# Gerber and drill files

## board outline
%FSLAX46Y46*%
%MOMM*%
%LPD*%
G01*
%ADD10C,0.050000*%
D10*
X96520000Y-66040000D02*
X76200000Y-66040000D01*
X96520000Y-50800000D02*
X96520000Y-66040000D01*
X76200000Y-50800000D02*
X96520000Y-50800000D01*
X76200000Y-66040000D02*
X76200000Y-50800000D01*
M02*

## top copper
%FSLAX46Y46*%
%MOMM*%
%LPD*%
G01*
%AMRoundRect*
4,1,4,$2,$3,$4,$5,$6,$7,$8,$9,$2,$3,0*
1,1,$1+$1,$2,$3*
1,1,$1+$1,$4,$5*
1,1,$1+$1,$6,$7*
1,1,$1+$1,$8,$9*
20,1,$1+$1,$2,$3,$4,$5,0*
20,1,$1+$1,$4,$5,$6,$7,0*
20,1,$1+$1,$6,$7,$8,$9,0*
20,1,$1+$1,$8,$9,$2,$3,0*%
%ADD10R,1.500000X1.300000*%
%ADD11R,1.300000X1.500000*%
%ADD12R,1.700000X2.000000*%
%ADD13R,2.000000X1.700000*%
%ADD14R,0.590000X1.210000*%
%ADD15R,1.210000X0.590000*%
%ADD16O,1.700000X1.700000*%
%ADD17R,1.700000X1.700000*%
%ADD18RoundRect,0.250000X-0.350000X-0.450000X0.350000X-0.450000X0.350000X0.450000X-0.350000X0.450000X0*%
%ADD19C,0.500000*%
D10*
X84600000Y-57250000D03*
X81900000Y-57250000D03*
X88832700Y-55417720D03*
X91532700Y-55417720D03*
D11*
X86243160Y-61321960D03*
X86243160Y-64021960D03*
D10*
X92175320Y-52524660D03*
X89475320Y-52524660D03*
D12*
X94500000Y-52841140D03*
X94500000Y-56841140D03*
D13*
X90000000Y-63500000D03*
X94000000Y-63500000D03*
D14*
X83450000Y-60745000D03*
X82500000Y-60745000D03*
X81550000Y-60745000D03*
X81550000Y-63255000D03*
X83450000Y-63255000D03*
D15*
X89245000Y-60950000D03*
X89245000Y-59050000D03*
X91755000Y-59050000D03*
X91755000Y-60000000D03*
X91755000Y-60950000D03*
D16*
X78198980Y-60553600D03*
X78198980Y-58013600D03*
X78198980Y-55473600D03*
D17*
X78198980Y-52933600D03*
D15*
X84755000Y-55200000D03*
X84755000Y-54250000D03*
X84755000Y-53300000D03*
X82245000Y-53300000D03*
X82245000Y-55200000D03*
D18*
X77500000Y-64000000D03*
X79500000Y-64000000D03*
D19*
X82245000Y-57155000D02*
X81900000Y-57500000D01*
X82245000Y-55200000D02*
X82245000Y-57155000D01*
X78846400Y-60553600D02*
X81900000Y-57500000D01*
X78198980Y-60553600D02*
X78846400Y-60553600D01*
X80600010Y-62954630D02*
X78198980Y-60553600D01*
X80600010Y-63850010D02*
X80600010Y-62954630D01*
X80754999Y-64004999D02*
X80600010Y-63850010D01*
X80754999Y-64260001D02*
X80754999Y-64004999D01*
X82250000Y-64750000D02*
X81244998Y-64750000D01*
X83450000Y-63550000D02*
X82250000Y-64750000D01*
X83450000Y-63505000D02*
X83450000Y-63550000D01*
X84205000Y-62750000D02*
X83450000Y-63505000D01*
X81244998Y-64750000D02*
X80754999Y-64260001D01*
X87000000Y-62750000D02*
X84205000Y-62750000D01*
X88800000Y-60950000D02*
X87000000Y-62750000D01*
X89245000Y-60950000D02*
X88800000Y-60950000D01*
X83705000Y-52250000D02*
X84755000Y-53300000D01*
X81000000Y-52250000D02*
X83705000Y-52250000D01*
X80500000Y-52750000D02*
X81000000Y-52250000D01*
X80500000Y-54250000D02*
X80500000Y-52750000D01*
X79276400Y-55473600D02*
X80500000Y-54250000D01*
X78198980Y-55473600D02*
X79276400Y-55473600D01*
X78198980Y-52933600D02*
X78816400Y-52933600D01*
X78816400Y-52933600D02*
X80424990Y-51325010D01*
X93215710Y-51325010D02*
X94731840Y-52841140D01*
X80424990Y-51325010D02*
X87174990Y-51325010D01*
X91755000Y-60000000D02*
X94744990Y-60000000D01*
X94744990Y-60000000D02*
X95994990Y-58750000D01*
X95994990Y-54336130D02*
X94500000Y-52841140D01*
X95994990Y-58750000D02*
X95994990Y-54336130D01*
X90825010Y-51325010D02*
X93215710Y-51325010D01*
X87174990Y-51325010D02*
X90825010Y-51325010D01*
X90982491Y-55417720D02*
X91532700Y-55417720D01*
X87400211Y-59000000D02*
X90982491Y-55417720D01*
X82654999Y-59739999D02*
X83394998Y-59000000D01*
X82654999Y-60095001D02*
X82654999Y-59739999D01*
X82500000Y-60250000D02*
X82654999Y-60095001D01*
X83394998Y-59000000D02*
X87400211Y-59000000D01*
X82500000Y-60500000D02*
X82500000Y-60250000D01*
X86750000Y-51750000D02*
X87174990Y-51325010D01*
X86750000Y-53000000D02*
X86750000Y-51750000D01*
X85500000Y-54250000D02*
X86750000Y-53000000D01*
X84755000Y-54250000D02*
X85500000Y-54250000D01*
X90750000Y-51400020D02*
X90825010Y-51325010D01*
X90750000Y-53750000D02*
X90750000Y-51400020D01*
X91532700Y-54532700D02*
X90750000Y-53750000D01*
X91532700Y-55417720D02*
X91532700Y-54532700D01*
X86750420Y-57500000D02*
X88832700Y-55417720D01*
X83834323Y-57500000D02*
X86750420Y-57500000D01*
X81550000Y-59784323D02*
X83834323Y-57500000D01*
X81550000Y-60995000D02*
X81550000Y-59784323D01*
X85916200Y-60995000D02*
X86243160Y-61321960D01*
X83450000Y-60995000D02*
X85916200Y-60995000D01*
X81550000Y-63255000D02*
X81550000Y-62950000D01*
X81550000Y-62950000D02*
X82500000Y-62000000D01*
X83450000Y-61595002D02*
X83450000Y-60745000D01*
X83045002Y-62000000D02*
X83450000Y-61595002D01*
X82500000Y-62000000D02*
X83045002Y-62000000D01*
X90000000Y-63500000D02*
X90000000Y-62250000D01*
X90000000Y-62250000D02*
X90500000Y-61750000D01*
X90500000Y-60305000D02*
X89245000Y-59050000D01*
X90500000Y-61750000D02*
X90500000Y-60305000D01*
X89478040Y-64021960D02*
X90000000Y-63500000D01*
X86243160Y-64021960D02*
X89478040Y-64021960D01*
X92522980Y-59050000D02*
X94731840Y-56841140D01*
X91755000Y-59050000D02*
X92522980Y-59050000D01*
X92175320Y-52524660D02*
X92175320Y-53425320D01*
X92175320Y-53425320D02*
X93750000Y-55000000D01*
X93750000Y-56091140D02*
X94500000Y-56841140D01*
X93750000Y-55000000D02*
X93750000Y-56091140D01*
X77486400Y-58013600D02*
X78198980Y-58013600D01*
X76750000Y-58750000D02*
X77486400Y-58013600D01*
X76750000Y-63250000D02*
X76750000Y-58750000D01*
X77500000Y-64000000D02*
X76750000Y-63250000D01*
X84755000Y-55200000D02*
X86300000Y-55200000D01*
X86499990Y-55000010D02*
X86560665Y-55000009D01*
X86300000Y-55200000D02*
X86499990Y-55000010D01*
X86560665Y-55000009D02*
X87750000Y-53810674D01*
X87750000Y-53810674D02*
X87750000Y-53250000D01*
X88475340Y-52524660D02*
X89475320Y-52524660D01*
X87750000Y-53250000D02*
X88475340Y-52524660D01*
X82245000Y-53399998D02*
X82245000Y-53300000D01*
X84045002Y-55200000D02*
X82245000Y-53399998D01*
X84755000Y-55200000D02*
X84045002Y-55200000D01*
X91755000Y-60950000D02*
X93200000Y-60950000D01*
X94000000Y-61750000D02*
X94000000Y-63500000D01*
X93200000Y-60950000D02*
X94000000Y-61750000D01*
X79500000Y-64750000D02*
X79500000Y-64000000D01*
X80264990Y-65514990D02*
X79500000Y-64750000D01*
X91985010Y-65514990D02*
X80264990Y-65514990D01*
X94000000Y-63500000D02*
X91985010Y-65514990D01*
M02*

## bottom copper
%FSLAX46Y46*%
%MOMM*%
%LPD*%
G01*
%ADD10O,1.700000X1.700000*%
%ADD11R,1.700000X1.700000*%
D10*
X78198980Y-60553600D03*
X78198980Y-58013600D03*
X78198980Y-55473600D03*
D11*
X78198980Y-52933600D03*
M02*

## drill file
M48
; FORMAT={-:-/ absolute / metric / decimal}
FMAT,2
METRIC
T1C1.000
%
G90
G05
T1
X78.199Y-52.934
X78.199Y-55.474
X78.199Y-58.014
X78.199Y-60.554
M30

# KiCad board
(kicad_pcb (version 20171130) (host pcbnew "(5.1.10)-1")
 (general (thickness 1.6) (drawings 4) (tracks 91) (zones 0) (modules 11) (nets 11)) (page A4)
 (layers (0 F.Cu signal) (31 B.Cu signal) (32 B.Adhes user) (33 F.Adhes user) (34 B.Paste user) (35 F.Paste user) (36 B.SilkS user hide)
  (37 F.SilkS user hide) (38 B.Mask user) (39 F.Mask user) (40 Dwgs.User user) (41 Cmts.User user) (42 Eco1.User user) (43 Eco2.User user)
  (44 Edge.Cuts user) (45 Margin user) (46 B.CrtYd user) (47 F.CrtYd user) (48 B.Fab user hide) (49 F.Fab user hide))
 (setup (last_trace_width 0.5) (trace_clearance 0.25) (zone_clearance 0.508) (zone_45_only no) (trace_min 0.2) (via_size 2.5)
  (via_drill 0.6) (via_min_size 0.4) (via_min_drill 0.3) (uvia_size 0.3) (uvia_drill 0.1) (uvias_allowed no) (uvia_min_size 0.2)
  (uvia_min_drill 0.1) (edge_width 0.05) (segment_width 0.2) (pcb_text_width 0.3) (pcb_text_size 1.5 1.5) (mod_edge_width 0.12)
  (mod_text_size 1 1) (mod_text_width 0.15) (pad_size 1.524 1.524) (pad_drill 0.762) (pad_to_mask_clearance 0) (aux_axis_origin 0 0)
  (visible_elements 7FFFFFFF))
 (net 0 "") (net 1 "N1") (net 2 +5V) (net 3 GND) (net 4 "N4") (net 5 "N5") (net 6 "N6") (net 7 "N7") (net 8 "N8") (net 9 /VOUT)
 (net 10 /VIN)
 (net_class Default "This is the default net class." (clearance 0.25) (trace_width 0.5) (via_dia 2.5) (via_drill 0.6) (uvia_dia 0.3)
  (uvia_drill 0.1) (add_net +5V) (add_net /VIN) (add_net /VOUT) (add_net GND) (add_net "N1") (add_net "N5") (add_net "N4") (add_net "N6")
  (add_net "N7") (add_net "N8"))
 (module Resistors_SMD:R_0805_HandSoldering (layer F.Cu) (at 83.25 57.25)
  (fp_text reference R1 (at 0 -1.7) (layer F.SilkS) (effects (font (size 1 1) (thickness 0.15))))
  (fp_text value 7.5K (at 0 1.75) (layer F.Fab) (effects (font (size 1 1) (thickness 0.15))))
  (pad 2 smd rect (at 1.35 0) (size 1.5 1.3) (layers F.Cu F.Paste F.Mask) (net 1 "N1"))
  (pad 1 smd rect (at -1.35 0) (size 1.5 1.3) (layers F.Cu F.Paste F.Mask) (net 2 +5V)))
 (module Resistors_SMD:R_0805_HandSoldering (layer F.Cu) (at 90.1827 55.41772)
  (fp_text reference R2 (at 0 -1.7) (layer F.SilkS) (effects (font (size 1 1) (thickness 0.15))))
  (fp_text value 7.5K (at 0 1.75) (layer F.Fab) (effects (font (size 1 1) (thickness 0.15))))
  (pad 1 smd rect (at -1.35 0) (size 1.5 1.3) (layers F.Cu F.Paste F.Mask) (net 1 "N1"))
  (pad 2 smd rect (at 1.35 0) (size 1.5 1.3) (layers F.Cu F.Paste F.Mask) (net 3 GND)))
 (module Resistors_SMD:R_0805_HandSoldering (layer F.Cu) (at 86.24316 62.67196 90)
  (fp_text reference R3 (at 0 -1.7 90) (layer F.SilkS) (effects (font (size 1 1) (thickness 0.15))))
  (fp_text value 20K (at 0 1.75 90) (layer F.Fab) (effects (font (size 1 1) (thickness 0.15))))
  (pad 2 smd rect (at 1.35 0 90) (size 1.5 1.3) (layers F.Cu F.Paste F.Mask) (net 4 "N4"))
  (pad 1 smd rect (at -1.35 0 90) (size 1.5 1.3) (layers F.Cu F.Paste F.Mask) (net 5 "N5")))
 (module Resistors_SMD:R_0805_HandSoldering (layer F.Cu) (at 90.82532 52.52466 180)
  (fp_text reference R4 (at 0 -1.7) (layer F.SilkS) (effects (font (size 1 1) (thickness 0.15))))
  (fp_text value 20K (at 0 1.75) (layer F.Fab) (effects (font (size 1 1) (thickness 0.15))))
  (pad 1 smd rect (at -1.35 0 180) (size 1.5 1.3) (layers F.Cu F.Paste F.Mask) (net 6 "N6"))
  (pad 2 smd rect (at 1.35 0 180) (size 1.5 1.3) (layers F.Cu F.Paste F.Mask) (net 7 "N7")))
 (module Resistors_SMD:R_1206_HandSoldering (layer F.Cu) (at 94.5 54.84114 270)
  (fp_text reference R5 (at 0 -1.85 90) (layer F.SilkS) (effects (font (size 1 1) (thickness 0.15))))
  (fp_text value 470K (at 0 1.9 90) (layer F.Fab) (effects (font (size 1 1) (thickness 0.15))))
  (pad 1 smd rect (at -2 0 270) (size 2 1.7) (layers F.Cu F.Paste F.Mask) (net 3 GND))
  (pad 2 smd rect (at 2 0 270) (size 2 1.7) (layers F.Cu F.Paste F.Mask) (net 6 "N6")))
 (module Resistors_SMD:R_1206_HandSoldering (layer F.Cu) (at 92 63.5 180)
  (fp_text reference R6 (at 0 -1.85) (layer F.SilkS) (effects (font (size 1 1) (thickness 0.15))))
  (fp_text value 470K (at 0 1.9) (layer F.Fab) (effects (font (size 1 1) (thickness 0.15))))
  (pad 2 smd rect (at 2 0 180) (size 2 1.7) (layers F.Cu F.Paste F.Mask) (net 5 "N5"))
  (pad 1 smd rect (at -2 0 180) (size 2 1.7) (layers F.Cu F.Paste F.Mask) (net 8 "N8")))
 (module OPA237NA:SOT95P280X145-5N (layer F.Cu) (at 82.5 62 270)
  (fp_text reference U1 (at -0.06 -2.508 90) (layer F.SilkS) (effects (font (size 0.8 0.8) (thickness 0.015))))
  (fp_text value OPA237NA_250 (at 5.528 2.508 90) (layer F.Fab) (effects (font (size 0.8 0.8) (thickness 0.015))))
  (pad 1 smd rect (at -1.255 -0.95 270) (size 1.21 0.59) (layers F.Cu F.Paste F.Mask) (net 4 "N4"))
  (pad 2 smd rect (at -1.255 0 270) (size 1.21 0.59) (layers F.Cu F.Paste F.Mask) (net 3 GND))
  (pad 3 smd rect (at -1.255 0.95 270) (size 1.21 0.59) (layers F.Cu F.Paste F.Mask) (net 1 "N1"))
  (pad 4 smd rect (at 1.255 0.95 270) (size 1.21 0.59) (layers F.Cu F.Paste F.Mask) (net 4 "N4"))
  (pad 5 smd rect (at 1.255 -0.95 270) (size 1.21 0.59) (layers F.Cu F.Paste F.Mask) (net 2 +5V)))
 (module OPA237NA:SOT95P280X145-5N (layer F.Cu) (at 90.5 60 180)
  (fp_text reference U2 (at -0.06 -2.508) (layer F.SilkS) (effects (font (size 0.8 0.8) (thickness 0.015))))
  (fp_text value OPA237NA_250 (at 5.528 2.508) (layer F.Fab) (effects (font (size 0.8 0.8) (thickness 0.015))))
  (pad 5 smd rect (at 1.255 -0.95 180) (size 1.21 0.59) (layers F.Cu F.Paste F.Mask) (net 2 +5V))
  (pad 4 smd rect (at 1.255 0.95 180) (size 1.21 0.59) (layers F.Cu F.Paste F.Mask) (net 5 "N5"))
  (pad 3 smd rect (at -1.255 0.95 180) (size 1.21 0.59) (layers F.Cu F.Paste F.Mask) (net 6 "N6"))
  (pad 2 smd rect (at -1.255 0 180) (size 1.21 0.59) (layers F.Cu F.Paste F.Mask) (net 3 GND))
  (pad 1 smd rect (at -1.255 -0.95 180) (size 1.21 0.59) (layers F.Cu F.Paste F.Mask) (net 8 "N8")))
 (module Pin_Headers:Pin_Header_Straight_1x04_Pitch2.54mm (layer F.Cu) (at 78.19898 52.9336)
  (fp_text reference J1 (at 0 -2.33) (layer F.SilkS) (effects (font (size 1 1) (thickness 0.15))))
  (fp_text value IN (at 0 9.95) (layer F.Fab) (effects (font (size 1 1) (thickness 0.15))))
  (pad 4 thru_hole oval (at 0 7.62) (size 1.7 1.7) (drill 1) (layers *.Cu *.Mask) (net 2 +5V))
  (pad 3 thru_hole oval (at 0 5.08) (size 1.7 1.7) (drill 1) (layers *.Cu *.Mask) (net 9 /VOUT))
  (pad 2 thru_hole oval (at 0 2.54) (size 1.7 1.7) (drill 1) (layers *.Cu *.Mask) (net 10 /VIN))
  (pad 1 thru_hole rect (at 0 0) (size 1.7 1.7) (drill 1) (layers *.Cu *.Mask) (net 3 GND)))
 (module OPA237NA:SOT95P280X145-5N (layer F.Cu) (at 83.5 54.25 180)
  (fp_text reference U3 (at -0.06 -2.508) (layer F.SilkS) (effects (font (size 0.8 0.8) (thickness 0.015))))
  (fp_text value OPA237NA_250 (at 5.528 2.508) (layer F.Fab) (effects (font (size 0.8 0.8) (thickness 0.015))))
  (pad 1 smd rect (at -1.255 -0.95 180) (size 1.21 0.59) (layers F.Cu F.Paste F.Mask) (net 7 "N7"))
  (pad 2 smd rect (at -1.255 0 180) (size 1.21 0.59) (layers F.Cu F.Paste F.Mask) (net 3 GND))
  (pad 3 smd rect (at -1.255 0.95 180) (size 1.21 0.59) (layers F.Cu F.Paste F.Mask) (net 10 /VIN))
  (pad 4 smd rect (at 1.255 0.95 180) (size 1.21 0.59) (layers F.Cu F.Paste F.Mask) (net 7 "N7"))
  (pad 5 smd rect (at 1.255 -0.95 180) (size 1.21 0.59) (layers F.Cu F.Paste F.Mask) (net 2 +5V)))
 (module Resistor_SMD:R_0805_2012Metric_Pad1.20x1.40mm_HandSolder (layer F.Cu) (at 78.5 64)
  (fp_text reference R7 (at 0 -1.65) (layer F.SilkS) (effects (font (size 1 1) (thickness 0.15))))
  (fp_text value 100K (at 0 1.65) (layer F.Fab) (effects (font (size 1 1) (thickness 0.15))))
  (pad 1 smd roundrect (at -1 0) (size 1.2 1.4) (layers F.Cu F.Paste F.Mask) (roundrect_rratio 0.208333) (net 9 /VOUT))
  (pad 2 smd roundrect (at 1 0) (size 1.2 1.4) (layers F.Cu F.Paste F.Mask) (roundrect_rratio 0.208333) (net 8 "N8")))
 (gr_line (start 96.52 66.04) (end 76.2 66.04) (layer Edge.Cuts) (width 0.05))
 (gr_line (start 96.52 50.8) (end 96.52 66.04) (layer Edge.Cuts) (width 0.05))
 (gr_line (start 76.2 50.8) (end 96.52 50.8) (layer Edge.Cuts) (width 0.05))
 (gr_line (start 76.2 66.04) (end 76.2 50.8) (layer Edge.Cuts) (width 0.05))
 (segment (start 82.245 57.155) (end 81.9 57.5) (width 0.5) (layer F.Cu) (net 2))
 (segment (start 82.245 55.2) (end 82.245 57.155) (width 0.5) (layer F.Cu) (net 2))
 (segment (start 78.8464 60.5536) (end 81.9 57.5) (width 0.5) (layer F.Cu) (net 2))
 (segment (start 78.19898 60.5536) (end 78.8464 60.5536) (width 0.5) (layer F.Cu) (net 2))
 (segment (start 80.60001 62.95463) (end 78.19898 60.5536) (width 0.5) (layer F.Cu) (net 2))
 (segment (start 80.60001 63.85001) (end 80.60001 62.95463) (width 0.5) (layer F.Cu) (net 2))
 (segment (start 80.754999 64.004999) (end 80.60001 63.85001) (width 0.5) (layer F.Cu) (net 2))
 (segment (start 80.754999 64.260001) (end 80.754999 64.004999) (width 0.5) (layer F.Cu) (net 2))
 (segment (start 82.25 64.75) (end 81.244998 64.75) (width 0.5) (layer F.Cu) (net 2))
 (segment (start 83.45 63.55) (end 82.25 64.75) (width 0.5) (layer F.Cu) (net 2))
 (segment (start 83.45 63.505) (end 83.45 63.55) (width 0.5) (layer F.Cu) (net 2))
 (segment (start 84.205 62.75) (end 83.45 63.505) (width 0.5) (layer F.Cu) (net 2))
 (segment (start 81.244998 64.75) (end 80.754999 64.260001) (width 0.5) (layer F.Cu) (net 2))
 (segment (start 87 62.75) (end 84.205 62.75) (width 0.5) (layer F.Cu) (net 2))
 (segment (start 88.8 60.95) (end 87 62.75) (width 0.5) (layer F.Cu) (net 2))
 (segment (start 89.245 60.95) (end 88.8 60.95) (width 0.5) (layer F.Cu) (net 2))
 (segment (start 83.705 52.25) (end 84.755 53.3) (width 0.5) (layer F.Cu) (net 10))
 (segment (start 81 52.25) (end 83.705 52.25) (width 0.5) (layer F.Cu) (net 10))
 (segment (start 80.5 52.75) (end 81 52.25) (width 0.5) (layer F.Cu) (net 10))
 (segment (start 80.5 54.25) (end 80.5 52.75) (width 0.5) (layer F.Cu) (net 10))
 (segment (start 79.2764 55.4736) (end 80.5 54.25) (width 0.5) (layer F.Cu) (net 10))
 (segment (start 78.19898 55.4736) (end 79.2764 55.4736) (width 0.5) (layer F.Cu) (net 10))
 (segment (start 78.19898 52.9336) (end 78.8164 52.9336) (width 0.5) (layer F.Cu) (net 3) (status 30))
 (segment (start 78.8164 52.9336) (end 80.42499 51.32501) (width 0.5) (layer F.Cu) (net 3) (status 10))
 (segment (start 93.21571 51.32501) (end 94.73184 52.84114) (width 0.5) (layer F.Cu) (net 3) (status 20))
 (segment (start 80.42499 51.32501) (end 87.17499 51.32501) (width 0.5) (layer F.Cu) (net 3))
 (segment (start 91.755 60) (end 94.74499 60) (width 0.5) (layer F.Cu) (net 3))
 (segment (start 94.74499 60) (end 95.99499 58.75) (width 0.5) (layer F.Cu) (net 3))
 (segment (start 95.99499 54.33613) (end 94.5 52.84114) (width 0.5) (layer F.Cu) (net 3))
 (segment (start 95.99499 58.75) (end 95.99499 54.33613) (width 0.5) (layer F.Cu) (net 3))
 (segment (start 90.82501 51.32501) (end 93.21571 51.32501) (width 0.5) (layer F.Cu) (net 3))
 (segment (start 87.17499 51.32501) (end 90.82501 51.32501) (width 0.5) (layer F.Cu) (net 3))
 (segment (start 90.982491 55.41772) (end 91.5327 55.41772) (width 0.5) (layer F.Cu) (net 3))
 (segment (start 87.400211 59) (end 90.982491 55.41772) (width 0.5) (layer F.Cu) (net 3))
 (segment (start 82.654999 59.739999) (end 83.394998 59) (width 0.5) (layer F.Cu) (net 3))
 (segment (start 82.654999 60.095001) (end 82.654999 59.739999) (width 0.5) (layer F.Cu) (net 3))
 (segment (start 82.5 60.25) (end 82.654999 60.095001) (width 0.5) (layer F.Cu) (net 3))
 (segment (start 83.394998 59) (end 87.400211 59) (width 0.5) (layer F.Cu) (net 3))
 (segment (start 82.5 60.5) (end 82.5 60.25) (width 0.5) (layer F.Cu) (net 3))
 (segment (start 86.75 51.75) (end 87.17499 51.32501) (width 0.5) (layer F.Cu) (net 3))
 (segment (start 86.75 53) (end 86.75 51.75) (width 0.5) (layer F.Cu) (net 3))
 (segment (start 85.5 54.25) (end 86.75 53) (width 0.5) (layer F.Cu) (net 3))
 (segment (start 84.755 54.25) (end 85.5 54.25) (width 0.5) (layer F.Cu) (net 3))
 (segment (start 90.75 51.40002) (end 90.82501 51.32501) (width 0.5) (layer F.Cu) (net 3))
 (segment (start 90.75 53.75) (end 90.75 51.40002) (width 0.5) (layer F.Cu) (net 3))
 (segment (start 91.5327 54.5327) (end 90.75 53.75) (width 0.5) (layer F.Cu) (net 3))
 (segment (start 91.5327 55.41772) (end 91.5327 54.5327) (width 0.5) (layer F.Cu) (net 3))
 (segment (start 86.75042 57.5) (end 88.8327 55.41772) (width 0.5) (layer F.Cu) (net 1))
 (segment (start 83.834323 57.5) (end 86.75042 57.5) (width 0.5) (layer F.Cu) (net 1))
 (segment (start 81.55 59.784323) (end 83.834323 57.5) (width 0.5) (layer F.Cu) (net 1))
 (segment (start 81.55 60.995) (end 81.55 59.784323) (width 0.5) (layer F.Cu) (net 1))
 (segment (start 85.9162 60.995) (end 86.24316 61.32196) (width 0.5) (layer F.Cu) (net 4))
 (segment (start 83.45 60.995) (end 85.9162 60.995) (width 0.5) (layer F.Cu) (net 4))
 (segment (start 81.55 63.255) (end 81.55 62.95) (width 0.5) (layer F.Cu) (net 4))
 (segment (start 81.55 62.95) (end 82.5 62) (width 0.5) (layer F.Cu) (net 4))
 (segment (start 83.45 61.595002) (end 83.45 60.745) (width 0.5) (layer F.Cu) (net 4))
 (segment (start 83.045002 62) (end 83.45 61.595002) (width 0.5) (layer F.Cu) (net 4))
 (segment (start 82.5 62) (end 83.045002 62) (width 0.5) (layer F.Cu) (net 4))
 (segment (start 90 63.5) (end 90 62.25) (width 0.5) (layer F.Cu) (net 5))
 (segment (start 90 62.25) (end 90.5 61.75) (width 0.5) (layer F.Cu) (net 5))
 (segment (start 90.5 60.305) (end 89.245 59.05) (width 0.5) (layer F.Cu) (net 5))
 (segment (start 90.5 61.75) (end 90.5 60.305) (width 0.5) (layer F.Cu) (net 5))
 (segment (start 89.47804 64.02196) (end 90 63.5) (width 0.5) (layer F.Cu) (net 5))
 (segment (start 86.24316 64.02196) (end 89.47804 64.02196) (width 0.5) (layer F.Cu) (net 5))
 (segment (start 92.52298 59.05) (end 94.73184 56.84114) (width 0.5) (layer F.Cu) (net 6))
 (segment (start 91.755 59.05) (end 92.52298 59.05) (width 0.5) (layer F.Cu) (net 6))
 (segment (start 92.17532 52.52466) (end 92.17532 53.42532) (width 0.5) (layer F.Cu) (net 6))
 (segment (start 92.17532 53.42532) (end 93.75 55) (width 0.5) (layer F.Cu) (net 6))
 (segment (start 93.75 56.09114) (end 94.5 56.84114) (width 0.5) (layer F.Cu) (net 6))
 (segment (start 93.75 55) (end 93.75 56.09114) (width 0.5) (layer F.Cu) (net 6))
 (segment (start 77.4864 58.0136) (end 78.19898 58.0136) (width 0.5) (layer F.Cu) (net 9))
 (segment (start 76.75 58.75) (end 77.4864 58.0136) (width 0.5) (layer F.Cu) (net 9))
 (segment (start 76.75 63.25) (end 76.75 58.75) (width 0.5) (layer F.Cu) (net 9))
 (segment (start 77.5 64) (end 76.75 63.25) (width 0.5) (layer F.Cu) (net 9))
 (segment (start 84.755 55.2) (end 86.3 55.2) (width 0.5) (layer F.Cu) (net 7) (status 10))
 (segment (start 86.49999 55.00001) (end 86.560665 55.000009) (width 0.5) (layer F.Cu) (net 7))
 (segment (start 86.3 55.2) (end 86.49999 55.00001) (width 0.5) (layer F.Cu) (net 7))
 (segment (start 86.560665 55.000009) (end 87.75 53.810674) (width 0.5) (layer F.Cu) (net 7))
 (segment (start 87.75 53.810674) (end 87.75 53.25) (width 0.5) (layer F.Cu) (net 7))
 (segment (start 88.47534 52.52466) (end 89.47532 52.52466) (width 0.5) (layer F.Cu) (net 7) (status 20))
 (segment (start 87.75 53.25) (end 88.47534 52.52466) (width 0.5) (layer F.Cu) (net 7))
 (segment (start 82.245 53.399998) (end 82.245 53.3) (width 0.5) (layer F.Cu) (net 7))
 (segment (start 84.045002 55.2) (end 82.245 53.399998) (width 0.5) (layer F.Cu) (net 7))
 (segment (start 84.755 55.2) (end 84.045002 55.2) (width 0.5) (layer F.Cu) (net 7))
 (segment (start 91.755 60.95) (end 93.2 60.95) (width 0.5) (layer F.Cu) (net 8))
 (segment (start 94 61.75) (end 94 63.5) (width 0.5) (layer F.Cu) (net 8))
 (segment (start 93.2 60.95) (end 94 61.75) (width 0.5) (layer F.Cu) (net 8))
 (segment (start 79.5 64.75) (end 79.5 64) (width 0.5) (layer F.Cu) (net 8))
 (segment (start 80.26499 65.51499) (end 79.5 64.75) (width 0.5) (layer F.Cu) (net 8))
 (segment (start 91.98501 65.51499) (end 80.26499 65.51499) (width 0.5) (layer F.Cu) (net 8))
 (segment (start 94 63.5) (end 91.98501 65.51499) (width 0.5) (layer F.Cu) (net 8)))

